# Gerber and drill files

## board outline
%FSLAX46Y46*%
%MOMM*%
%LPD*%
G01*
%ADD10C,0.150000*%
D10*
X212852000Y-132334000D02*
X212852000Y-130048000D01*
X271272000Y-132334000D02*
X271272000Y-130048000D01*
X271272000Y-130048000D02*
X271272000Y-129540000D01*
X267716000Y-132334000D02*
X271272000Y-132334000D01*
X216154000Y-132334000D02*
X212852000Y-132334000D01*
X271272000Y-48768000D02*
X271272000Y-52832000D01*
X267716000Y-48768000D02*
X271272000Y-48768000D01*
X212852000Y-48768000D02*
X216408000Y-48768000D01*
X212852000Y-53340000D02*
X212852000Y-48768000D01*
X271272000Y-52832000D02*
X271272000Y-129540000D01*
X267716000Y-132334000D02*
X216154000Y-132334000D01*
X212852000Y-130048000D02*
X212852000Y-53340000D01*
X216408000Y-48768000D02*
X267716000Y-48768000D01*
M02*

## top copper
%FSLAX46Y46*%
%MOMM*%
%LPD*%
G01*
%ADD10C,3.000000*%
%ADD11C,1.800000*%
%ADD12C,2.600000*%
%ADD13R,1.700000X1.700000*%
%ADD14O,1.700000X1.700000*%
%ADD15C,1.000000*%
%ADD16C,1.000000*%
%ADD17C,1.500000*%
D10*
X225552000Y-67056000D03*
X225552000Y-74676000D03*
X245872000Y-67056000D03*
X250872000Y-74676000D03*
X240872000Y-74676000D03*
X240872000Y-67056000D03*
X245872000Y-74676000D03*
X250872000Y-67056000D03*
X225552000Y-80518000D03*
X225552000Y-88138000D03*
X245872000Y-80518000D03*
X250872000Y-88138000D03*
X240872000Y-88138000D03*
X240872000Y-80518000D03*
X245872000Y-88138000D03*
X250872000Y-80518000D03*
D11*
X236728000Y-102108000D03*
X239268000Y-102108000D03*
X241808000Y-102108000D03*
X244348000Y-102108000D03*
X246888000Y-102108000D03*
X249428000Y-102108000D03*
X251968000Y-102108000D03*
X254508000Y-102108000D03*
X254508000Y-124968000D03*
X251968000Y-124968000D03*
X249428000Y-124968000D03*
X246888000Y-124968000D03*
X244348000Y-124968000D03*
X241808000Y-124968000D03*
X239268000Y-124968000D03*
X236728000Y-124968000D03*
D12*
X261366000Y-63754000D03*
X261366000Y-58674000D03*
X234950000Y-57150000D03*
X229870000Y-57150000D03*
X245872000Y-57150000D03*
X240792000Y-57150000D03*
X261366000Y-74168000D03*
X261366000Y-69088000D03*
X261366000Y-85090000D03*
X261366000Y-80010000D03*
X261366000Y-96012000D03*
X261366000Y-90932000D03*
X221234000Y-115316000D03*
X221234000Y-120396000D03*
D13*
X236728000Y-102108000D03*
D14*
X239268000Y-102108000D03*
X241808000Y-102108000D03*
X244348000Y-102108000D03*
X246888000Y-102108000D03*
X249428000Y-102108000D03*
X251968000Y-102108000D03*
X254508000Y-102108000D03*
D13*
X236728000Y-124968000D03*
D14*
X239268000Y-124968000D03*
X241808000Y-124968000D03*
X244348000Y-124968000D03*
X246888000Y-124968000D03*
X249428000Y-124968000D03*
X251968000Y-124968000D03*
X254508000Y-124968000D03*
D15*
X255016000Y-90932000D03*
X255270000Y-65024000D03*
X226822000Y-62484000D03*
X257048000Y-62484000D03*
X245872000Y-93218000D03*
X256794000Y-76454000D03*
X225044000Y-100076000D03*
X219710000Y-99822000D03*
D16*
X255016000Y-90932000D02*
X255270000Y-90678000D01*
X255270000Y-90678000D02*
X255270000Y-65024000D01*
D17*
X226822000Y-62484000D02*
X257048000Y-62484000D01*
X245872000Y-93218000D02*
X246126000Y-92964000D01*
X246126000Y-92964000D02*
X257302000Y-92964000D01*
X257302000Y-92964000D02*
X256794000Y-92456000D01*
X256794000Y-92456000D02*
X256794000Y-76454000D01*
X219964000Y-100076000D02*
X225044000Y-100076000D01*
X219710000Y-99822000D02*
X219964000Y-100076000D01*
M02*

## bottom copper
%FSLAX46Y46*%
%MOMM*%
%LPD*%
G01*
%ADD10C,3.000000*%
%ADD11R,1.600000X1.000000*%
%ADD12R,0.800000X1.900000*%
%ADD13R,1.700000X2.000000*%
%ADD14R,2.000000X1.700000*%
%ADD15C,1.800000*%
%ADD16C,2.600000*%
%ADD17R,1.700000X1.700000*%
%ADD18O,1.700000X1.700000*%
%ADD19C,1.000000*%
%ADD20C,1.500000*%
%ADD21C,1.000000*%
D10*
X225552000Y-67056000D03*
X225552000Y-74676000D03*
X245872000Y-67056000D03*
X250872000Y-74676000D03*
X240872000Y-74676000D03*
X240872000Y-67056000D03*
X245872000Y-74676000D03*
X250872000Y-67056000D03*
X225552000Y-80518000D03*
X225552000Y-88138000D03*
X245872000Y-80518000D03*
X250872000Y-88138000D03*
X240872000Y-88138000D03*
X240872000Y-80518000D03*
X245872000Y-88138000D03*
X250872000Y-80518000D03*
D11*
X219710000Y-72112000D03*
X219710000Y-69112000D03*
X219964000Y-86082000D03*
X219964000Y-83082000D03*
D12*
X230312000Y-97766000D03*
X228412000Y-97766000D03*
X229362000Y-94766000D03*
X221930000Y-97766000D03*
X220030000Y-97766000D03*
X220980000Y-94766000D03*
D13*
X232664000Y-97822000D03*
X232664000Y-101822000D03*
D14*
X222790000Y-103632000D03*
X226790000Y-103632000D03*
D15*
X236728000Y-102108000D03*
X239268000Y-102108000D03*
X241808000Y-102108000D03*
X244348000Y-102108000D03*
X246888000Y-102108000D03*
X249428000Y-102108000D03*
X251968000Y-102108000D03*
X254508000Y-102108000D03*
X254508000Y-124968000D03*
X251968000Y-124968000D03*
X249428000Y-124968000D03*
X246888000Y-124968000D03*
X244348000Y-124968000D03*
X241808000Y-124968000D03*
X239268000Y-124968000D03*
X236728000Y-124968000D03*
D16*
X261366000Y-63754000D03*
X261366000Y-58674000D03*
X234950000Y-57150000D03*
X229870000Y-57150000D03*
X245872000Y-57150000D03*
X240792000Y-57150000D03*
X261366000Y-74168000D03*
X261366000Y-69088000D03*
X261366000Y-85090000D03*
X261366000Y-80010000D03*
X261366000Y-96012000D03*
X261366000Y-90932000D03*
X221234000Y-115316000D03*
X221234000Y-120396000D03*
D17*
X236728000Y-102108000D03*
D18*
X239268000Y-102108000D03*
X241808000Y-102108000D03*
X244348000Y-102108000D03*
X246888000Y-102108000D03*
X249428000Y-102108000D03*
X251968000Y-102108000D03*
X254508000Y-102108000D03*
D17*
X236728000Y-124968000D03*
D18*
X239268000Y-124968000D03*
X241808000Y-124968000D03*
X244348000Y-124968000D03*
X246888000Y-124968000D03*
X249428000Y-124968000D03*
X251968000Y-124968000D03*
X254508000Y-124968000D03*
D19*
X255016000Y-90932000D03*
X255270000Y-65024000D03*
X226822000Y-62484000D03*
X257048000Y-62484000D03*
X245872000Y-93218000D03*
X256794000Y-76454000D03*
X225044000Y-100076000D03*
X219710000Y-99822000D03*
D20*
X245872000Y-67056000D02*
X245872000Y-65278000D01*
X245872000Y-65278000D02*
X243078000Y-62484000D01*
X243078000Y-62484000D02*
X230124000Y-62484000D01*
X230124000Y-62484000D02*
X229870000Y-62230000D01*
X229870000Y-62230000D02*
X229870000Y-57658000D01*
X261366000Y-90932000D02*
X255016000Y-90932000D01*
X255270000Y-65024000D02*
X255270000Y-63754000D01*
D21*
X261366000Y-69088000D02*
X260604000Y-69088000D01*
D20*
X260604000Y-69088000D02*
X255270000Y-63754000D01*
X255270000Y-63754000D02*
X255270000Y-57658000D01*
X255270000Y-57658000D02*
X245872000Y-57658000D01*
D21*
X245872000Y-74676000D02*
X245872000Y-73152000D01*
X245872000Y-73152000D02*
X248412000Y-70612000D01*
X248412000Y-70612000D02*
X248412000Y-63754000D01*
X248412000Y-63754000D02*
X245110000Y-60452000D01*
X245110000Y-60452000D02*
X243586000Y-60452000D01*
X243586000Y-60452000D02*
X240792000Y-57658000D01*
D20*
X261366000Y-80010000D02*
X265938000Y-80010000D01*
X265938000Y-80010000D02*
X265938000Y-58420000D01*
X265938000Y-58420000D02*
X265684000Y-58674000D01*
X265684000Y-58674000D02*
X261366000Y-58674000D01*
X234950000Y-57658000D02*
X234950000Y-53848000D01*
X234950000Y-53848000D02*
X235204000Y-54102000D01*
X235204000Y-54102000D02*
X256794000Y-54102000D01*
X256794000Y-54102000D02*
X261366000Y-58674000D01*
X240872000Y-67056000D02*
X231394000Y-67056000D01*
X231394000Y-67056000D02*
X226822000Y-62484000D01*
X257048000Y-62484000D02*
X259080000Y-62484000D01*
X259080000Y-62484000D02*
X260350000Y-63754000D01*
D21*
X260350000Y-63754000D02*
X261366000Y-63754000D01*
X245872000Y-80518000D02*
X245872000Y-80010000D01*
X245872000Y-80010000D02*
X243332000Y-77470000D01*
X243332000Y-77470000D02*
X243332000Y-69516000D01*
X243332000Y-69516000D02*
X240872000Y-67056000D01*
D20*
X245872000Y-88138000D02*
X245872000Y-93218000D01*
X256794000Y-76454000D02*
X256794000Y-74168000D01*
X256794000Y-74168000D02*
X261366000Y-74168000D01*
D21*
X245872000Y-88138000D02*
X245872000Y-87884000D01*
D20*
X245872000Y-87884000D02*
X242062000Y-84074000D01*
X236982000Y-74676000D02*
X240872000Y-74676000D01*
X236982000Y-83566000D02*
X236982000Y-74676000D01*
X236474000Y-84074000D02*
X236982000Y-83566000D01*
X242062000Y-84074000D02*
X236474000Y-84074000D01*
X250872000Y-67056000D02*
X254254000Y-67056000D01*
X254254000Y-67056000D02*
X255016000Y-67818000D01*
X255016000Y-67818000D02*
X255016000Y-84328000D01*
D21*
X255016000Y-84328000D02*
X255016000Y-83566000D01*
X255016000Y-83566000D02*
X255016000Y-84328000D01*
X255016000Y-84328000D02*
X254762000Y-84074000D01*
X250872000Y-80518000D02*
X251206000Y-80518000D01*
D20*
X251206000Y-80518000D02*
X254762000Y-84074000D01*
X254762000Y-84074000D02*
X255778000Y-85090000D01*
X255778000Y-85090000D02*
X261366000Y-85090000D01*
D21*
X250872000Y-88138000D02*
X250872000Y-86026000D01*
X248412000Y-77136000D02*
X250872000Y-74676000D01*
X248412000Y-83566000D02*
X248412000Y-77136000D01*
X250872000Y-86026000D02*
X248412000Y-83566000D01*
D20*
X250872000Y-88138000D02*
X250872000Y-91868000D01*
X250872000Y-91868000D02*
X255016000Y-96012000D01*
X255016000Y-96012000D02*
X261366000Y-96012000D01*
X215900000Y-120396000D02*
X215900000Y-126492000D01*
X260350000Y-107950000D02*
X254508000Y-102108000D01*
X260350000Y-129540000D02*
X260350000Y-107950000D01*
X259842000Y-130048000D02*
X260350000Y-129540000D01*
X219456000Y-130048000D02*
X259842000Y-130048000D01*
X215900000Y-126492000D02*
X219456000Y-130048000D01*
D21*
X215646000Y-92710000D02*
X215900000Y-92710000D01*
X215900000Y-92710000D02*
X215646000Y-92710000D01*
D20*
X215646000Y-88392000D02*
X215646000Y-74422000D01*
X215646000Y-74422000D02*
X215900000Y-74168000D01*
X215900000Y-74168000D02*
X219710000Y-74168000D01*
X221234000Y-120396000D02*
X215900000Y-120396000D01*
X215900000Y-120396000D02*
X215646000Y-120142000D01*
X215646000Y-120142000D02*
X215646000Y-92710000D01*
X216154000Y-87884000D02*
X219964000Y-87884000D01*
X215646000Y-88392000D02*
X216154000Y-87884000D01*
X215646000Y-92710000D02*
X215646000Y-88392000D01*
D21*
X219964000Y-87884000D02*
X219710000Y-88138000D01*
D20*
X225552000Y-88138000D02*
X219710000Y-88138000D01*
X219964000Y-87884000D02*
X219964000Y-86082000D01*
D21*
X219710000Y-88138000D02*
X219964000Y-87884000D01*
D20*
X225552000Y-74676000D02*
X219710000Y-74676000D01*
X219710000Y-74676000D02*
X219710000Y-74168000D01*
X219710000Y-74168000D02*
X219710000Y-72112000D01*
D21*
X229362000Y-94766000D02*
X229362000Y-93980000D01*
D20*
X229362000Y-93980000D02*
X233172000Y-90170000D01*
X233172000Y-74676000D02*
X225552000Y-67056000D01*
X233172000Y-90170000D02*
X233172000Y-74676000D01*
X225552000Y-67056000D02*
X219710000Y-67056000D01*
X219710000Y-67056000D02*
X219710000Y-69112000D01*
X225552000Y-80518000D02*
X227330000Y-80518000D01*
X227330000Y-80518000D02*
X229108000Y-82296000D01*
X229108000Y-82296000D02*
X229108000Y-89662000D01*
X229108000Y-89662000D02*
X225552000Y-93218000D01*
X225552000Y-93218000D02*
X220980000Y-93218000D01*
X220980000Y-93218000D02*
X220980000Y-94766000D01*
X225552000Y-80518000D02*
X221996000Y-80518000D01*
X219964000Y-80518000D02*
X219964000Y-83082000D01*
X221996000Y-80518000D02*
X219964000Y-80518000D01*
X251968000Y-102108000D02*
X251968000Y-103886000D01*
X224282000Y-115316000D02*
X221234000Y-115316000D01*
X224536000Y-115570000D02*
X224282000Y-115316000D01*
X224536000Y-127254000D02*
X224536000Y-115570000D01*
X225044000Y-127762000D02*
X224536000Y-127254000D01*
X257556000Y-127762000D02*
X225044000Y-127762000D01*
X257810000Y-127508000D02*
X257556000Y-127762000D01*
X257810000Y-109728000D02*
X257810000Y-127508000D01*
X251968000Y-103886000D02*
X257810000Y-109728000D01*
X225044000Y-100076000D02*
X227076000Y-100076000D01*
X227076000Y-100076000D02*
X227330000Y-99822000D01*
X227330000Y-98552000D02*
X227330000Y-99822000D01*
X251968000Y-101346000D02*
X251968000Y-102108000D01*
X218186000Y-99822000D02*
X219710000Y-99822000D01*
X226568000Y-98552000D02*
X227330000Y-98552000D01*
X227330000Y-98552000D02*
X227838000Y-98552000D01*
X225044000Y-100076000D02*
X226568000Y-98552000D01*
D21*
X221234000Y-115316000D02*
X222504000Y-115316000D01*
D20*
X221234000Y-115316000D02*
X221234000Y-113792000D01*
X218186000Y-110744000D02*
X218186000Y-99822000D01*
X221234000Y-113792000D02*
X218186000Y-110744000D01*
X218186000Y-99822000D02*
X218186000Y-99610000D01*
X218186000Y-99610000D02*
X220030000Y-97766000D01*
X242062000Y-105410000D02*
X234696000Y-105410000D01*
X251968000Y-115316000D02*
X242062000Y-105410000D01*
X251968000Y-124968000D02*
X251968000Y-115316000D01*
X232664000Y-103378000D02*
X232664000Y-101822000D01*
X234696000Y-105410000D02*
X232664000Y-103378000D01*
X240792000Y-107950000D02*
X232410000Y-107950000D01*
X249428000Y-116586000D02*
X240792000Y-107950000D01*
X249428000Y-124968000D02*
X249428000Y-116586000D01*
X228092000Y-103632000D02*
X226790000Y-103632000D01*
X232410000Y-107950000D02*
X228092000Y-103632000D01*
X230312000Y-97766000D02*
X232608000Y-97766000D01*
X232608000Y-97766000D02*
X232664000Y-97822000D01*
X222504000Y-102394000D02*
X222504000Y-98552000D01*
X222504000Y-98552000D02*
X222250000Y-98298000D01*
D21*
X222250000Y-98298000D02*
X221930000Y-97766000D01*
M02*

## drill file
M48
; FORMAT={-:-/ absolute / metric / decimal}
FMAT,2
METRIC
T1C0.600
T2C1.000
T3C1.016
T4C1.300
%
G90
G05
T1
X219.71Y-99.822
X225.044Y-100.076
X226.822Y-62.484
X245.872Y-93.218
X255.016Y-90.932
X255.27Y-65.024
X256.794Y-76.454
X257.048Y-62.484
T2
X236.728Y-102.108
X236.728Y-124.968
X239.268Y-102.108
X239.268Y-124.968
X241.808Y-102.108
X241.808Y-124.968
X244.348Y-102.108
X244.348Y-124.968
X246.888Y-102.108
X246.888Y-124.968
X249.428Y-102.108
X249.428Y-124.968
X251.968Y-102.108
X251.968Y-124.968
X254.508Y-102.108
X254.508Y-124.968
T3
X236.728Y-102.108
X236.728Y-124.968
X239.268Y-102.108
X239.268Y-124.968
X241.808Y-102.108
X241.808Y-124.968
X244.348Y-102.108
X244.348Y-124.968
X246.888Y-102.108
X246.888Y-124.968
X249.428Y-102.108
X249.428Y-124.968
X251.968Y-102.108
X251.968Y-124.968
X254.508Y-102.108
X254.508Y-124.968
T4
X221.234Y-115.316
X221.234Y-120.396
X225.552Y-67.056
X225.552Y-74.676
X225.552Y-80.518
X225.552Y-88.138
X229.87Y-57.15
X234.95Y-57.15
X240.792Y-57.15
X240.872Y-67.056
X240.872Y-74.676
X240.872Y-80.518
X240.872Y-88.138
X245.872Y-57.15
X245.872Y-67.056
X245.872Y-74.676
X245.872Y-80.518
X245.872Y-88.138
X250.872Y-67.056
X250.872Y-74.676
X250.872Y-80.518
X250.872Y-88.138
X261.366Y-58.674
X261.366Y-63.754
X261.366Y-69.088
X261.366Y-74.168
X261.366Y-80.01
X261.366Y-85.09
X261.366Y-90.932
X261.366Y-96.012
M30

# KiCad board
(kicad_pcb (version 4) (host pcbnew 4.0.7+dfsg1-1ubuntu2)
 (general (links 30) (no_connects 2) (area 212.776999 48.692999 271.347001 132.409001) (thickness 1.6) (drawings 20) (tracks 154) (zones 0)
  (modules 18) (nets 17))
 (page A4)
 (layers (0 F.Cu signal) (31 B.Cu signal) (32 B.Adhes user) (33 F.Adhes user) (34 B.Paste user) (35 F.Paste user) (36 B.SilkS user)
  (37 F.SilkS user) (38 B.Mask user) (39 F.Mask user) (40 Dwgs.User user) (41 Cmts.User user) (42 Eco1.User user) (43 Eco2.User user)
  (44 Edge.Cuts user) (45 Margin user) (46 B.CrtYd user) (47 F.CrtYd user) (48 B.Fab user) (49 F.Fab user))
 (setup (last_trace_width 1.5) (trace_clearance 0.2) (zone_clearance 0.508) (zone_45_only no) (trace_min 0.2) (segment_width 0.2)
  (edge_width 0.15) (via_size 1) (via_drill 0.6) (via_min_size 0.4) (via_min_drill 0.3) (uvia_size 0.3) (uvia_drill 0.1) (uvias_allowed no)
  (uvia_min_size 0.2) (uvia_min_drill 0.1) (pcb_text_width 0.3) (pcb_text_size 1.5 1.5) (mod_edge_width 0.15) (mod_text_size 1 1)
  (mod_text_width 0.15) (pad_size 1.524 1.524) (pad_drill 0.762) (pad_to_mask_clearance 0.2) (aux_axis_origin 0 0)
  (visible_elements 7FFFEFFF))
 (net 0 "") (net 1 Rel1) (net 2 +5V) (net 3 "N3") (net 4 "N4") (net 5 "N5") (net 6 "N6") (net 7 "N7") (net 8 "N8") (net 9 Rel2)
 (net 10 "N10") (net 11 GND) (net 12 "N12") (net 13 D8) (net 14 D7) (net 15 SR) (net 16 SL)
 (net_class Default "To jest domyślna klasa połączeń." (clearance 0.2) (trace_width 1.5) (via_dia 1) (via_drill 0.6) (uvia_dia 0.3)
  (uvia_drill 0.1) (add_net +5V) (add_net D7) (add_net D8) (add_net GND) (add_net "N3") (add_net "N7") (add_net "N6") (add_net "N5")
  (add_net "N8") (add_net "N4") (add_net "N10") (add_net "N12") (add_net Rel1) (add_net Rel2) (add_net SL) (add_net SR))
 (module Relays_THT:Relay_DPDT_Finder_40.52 (layer F.Cu) (at 225.552 67.056)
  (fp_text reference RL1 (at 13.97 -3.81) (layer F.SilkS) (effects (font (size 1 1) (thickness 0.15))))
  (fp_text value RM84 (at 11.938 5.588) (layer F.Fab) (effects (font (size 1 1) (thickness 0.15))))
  (pad A1 thru_hole circle (at 0 0) (size 3 3) (drill 1.3) (layers *.Cu *.Mask) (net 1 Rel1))
  (pad A2 thru_hole circle (at 0 7.62) (size 3 3) (drill 1.3) (layers *.Cu *.Mask) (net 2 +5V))
  (pad 11 thru_hole circle (at 20.32 0) (size 3 3) (drill 1.3) (layers *.Cu *.Mask) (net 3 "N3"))
  (pad 24 thru_hole circle (at 25.32 7.62) (size 3 3) (drill 1.3) (layers *.Cu *.Mask) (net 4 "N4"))
  (pad 22 thru_hole circle (at 15.32 7.62) (size 3 3) (drill 1.3) (layers *.Cu *.Mask) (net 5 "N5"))
  (pad 12 thru_hole circle (at 15.32 0) (size 3 3) (drill 1.3) (layers *.Cu *.Mask) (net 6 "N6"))
  (pad 21 thru_hole circle (at 20.32 7.62) (size 3 3) (drill 1.3) (layers *.Cu *.Mask) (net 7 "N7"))
  (pad 14 thru_hole circle (at 25.32 0) (size 3 3) (drill 1.3) (layers *.Cu *.Mask) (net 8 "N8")))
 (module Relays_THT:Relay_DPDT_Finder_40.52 (layer F.Cu) (at 225.552 80.518)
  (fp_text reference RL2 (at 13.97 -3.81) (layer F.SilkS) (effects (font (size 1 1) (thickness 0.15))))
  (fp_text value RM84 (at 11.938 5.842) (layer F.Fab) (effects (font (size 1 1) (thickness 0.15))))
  (pad A1 thru_hole circle (at 0 0) (size 3 3) (drill 1.3) (layers *.Cu *.Mask) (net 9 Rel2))
  (pad A2 thru_hole circle (at 0 7.62) (size 3 3) (drill 1.3) (layers *.Cu *.Mask) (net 2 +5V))
  (pad 11 thru_hole circle (at 20.32 0) (size 3 3) (drill 1.3) (layers *.Cu *.Mask) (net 6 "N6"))
  (pad 24 thru_hole circle (at 25.32 7.62) (size 3 3) (drill 1.3) (layers *.Cu *.Mask) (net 4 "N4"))
  (pad 22 thru_hole circle (at 15.32 7.62) (size 3 3) (drill 1.3) (layers *.Cu *.Mask))
  (pad 12 thru_hole circle (at 15.32 0) (size 3 3) (drill 1.3) (layers *.Cu *.Mask))
  (pad 21 thru_hole circle (at 20.32 7.62) (size 3 3) (drill 1.3) (layers *.Cu *.Mask) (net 5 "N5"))
  (pad 14 thru_hole circle (at 25.32 0) (size 3 3) (drill 1.3) (layers *.Cu *.Mask) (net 8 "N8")))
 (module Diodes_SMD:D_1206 (layer B.Cu) (at 219.71 70.612 90)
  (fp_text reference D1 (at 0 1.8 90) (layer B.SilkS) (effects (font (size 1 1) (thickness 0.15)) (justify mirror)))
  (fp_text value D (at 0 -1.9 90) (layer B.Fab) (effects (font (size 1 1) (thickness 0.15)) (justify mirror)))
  (pad 1 smd rect (at -1.5 0 90) (size 1 1.6) (layers B.Cu B.Paste B.Mask) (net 2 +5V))
  (pad 2 smd rect (at 1.5 0 90) (size 1 1.6) (layers B.Cu B.Paste B.Mask) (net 1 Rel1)))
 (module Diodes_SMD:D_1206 (layer B.Cu) (at 219.964 84.582 90)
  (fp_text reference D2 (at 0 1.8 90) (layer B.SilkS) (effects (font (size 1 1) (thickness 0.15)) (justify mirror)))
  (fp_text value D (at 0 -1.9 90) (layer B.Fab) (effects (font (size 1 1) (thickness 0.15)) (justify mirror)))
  (pad 1 smd rect (at -1.5 0 90) (size 1 1.6) (layers B.Cu B.Paste B.Mask) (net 2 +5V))
  (pad 2 smd rect (at 1.5 0 90) (size 1 1.6) (layers B.Cu B.Paste B.Mask) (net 9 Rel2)))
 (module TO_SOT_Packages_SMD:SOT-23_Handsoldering (layer B.Cu) (at 229.362 96.266 90)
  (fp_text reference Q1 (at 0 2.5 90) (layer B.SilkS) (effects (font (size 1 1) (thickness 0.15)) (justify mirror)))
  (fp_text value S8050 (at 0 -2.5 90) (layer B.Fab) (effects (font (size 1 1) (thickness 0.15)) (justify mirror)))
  (pad 1 smd rect (at -1.5 0.95 90) (size 1.9 0.8) (layers B.Cu B.Paste B.Mask) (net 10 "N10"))
  (pad 2 smd rect (at -1.5 -0.95 90) (size 1.9 0.8) (layers B.Cu B.Paste B.Mask) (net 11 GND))
  (pad 3 smd rect (at 1.5 0 90) (size 1.9 0.8) (layers B.Cu B.Paste B.Mask) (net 1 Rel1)))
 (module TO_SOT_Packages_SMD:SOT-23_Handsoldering (layer B.Cu) (at 220.98 96.266 90)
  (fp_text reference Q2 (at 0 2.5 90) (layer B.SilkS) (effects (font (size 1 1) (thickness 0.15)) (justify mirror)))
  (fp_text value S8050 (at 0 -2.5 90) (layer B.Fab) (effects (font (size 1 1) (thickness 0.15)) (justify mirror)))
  (pad 1 smd rect (at -1.5 0.95 90) (size 1.9 0.8) (layers B.Cu B.Paste B.Mask) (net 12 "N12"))
  (pad 2 smd rect (at -1.5 -0.95 90) (size 1.9 0.8) (layers B.Cu B.Paste B.Mask) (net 11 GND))
  (pad 3 smd rect (at 1.5 0 90) (size 1.9 0.8) (layers B.Cu B.Paste B.Mask) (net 9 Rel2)))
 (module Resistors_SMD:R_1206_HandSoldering (layer B.Cu) (at 232.664 99.822 270)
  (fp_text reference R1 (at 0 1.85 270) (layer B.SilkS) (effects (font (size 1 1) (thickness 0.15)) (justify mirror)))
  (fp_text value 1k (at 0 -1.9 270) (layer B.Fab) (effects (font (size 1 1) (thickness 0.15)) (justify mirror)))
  (pad 1 smd rect (at -2 0 270) (size 2 1.7) (layers B.Cu B.Paste B.Mask) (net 10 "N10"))
  (pad 2 smd rect (at 2 0 270) (size 2 1.7) (layers B.Cu B.Paste B.Mask) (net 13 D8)))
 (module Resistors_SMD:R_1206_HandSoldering (layer B.Cu) (at 224.79 103.632)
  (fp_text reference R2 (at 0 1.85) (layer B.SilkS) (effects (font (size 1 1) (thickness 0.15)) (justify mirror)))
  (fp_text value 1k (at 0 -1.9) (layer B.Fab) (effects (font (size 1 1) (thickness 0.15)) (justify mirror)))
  (pad 1 smd rect (at -2 0) (size 2 1.7) (layers B.Cu B.Paste B.Mask) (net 12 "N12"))
  (pad 2 smd rect (at 2 0) (size 2 1.7) (layers B.Cu B.Paste B.Mask) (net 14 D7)))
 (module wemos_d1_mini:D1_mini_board (layer B.Cu) (at 246.888 113.538 270)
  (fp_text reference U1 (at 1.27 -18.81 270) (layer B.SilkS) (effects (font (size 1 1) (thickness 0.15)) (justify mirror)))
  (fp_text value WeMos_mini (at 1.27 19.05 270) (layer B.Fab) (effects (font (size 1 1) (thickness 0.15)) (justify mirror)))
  (pad 8 thru_hole circle (at -11.43 10.16 270) (size 1.8 1.8) (drill 1.016) (layers *.Cu *.Mask B.SilkS))
  (pad 7 thru_hole circle (at -11.43 7.62 270) (size 1.8 1.8) (drill 1.016) (layers *.Cu *.Mask B.SilkS))
  (pad 6 thru_hole circle (at -11.43 5.08 270) (size 1.8 1.8) (drill 1.016) (layers *.Cu *.Mask B.SilkS))
  (pad 5 thru_hole circle (at -11.43 2.54 270) (size 1.8 1.8) (drill 1.016) (layers *.Cu *.Mask B.SilkS))
  (pad 4 thru_hole circle (at -11.43 0 270) (size 1.8 1.8) (drill 1.016) (layers *.Cu *.Mask B.SilkS))
  (pad 3 thru_hole circle (at -11.43 -2.54 270) (size 1.8 1.8) (drill 1.016) (layers *.Cu *.Mask B.SilkS))
  (pad 2 thru_hole circle (at -11.43 -5.08 270) (size 1.8 1.8) (drill 1.016) (layers *.Cu *.Mask B.SilkS) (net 11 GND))
  (pad 1 thru_hole circle (at -11.43 -7.62 270) (size 1.8 1.8) (drill 1.016) (layers *.Cu *.Mask B.SilkS) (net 2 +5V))
  (pad 16 thru_hole circle (at 11.43 -7.62 270) (size 1.8 1.8) (drill 1.016) (layers *.Cu *.Mask B.SilkS))
  (pad 15 thru_hole circle (at 11.43 -5.08 270) (size 1.8 1.8) (drill 1.016) (layers *.Cu *.Mask B.SilkS) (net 13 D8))
  (pad 14 thru_hole circle (at 11.43 -2.54 270) (size 1.8 1.8) (drill 1.016) (layers *.Cu *.Mask B.SilkS) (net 14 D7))
  (pad 13 thru_hole circle (at 11.43 0 270) (size 1.8 1.8) (drill 1.016) (layers *.Cu *.Mask B.SilkS))
  (pad 12 thru_hole circle (at 11.43 2.54 270) (size 1.8 1.8) (drill 1.016) (layers *.Cu *.Mask B.SilkS))
  (pad 11 thru_hole circle (at 11.43 5.08 270) (size 1.8 1.8) (drill 1.016) (layers *.Cu *.Mask B.SilkS))
  (pad 10 thru_hole circle (at 11.43 7.62 270) (size 1.8 1.8) (drill 1.016) (layers *.Cu *.Mask B.SilkS))
  (pad 9 thru_hole circle (at 11.43 10.16 270) (size 1.8 1.8) (drill 1.016) (layers *.Cu *.Mask B.SilkS)))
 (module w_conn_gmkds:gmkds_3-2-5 (layer F.Cu) (at 261.366 61.214 90)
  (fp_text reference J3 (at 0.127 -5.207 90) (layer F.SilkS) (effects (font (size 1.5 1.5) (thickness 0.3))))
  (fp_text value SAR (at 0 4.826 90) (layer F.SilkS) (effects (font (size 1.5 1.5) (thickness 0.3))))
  (pad 1 thru_hole circle (at -2.54 0 90) (size 2.6 2.6) (drill 1.3) (layers *.Cu *.Mask F.SilkS) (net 6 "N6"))
  (pad 2 thru_hole circle (at 2.54 0 90) (size 2.6 2.6) (drill 1.3) (layers *.Cu *.Mask F.SilkS) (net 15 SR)))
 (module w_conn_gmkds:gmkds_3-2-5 (layer F.Cu) (at 232.41 57.15 180)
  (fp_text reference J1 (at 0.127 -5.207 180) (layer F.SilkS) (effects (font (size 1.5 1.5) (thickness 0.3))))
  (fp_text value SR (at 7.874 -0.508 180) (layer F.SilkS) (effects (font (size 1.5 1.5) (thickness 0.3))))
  (pad 1 thru_hole circle (at -2.54 0 180) (size 2.6 2.6) (drill 1.3) (layers *.Cu *.Mask F.SilkS) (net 15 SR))
  (pad 2 thru_hole circle (at 2.54 0 180) (size 2.6 2.6) (drill 1.3) (layers *.Cu *.Mask F.SilkS) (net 3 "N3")))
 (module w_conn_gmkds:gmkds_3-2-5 (layer F.Cu) (at 243.332 57.15 180)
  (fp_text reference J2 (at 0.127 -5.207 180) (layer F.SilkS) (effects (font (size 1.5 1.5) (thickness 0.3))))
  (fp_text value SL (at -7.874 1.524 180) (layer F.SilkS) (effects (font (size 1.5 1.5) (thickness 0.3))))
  (pad 1 thru_hole circle (at -2.54 0 180) (size 2.6 2.6) (drill 1.3) (layers *.Cu *.Mask F.SilkS) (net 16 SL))
  (pad 2 thru_hole circle (at 2.54 0 180) (size 2.6 2.6) (drill 1.3) (layers *.Cu *.Mask F.SilkS) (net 7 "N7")))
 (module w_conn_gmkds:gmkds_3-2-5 (layer F.Cu) (at 261.366 71.628 90)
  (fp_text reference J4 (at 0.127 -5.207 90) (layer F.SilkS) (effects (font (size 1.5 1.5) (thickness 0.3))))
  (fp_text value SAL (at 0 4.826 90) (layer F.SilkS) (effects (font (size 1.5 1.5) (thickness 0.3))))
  (pad 1 thru_hole circle (at -2.54 0 90) (size 2.6 2.6) (drill 1.3) (layers *.Cu *.Mask F.SilkS) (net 5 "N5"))
  (pad 2 thru_hole circle (at 2.54 0 90) (size 2.6 2.6) (drill 1.3) (layers *.Cu *.Mask F.SilkS) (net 16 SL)))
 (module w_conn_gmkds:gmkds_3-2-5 (layer F.Cu) (at 261.366 82.55 90)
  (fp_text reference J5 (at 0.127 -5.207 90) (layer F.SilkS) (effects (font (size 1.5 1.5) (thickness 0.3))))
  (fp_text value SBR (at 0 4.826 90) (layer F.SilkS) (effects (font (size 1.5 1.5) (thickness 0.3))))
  (pad 1 thru_hole circle (at -2.54 0 90) (size 2.6 2.6) (drill 1.3) (layers *.Cu *.Mask F.SilkS) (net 8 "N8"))
  (pad 2 thru_hole circle (at 2.54 0 90) (size 2.6 2.6) (drill 1.3) (layers *.Cu *.Mask F.SilkS) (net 15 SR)))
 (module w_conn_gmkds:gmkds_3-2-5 (layer F.Cu) (at 261.366 93.472 90)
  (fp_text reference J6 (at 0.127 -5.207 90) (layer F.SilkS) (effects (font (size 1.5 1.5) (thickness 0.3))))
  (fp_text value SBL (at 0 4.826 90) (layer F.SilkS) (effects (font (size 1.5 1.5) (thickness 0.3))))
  (pad 1 thru_hole circle (at -2.54 0 90) (size 2.6 2.6) (drill 1.3) (layers *.Cu *.Mask F.SilkS) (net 4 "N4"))
  (pad 2 thru_hole circle (at 2.54 0 90) (size 2.6 2.6) (drill 1.3) (layers *.Cu *.Mask F.SilkS) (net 16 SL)))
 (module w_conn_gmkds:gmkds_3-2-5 (layer F.Cu) (at 221.234 117.856 270)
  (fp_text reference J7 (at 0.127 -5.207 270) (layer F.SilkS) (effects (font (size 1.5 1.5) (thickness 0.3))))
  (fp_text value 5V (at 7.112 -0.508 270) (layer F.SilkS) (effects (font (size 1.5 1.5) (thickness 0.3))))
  (pad 1 thru_hole circle (at -2.54 0 270) (size 2.6 2.6) (drill 1.3) (layers *.Cu *.Mask F.SilkS) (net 11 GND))
  (pad 2 thru_hole circle (at 2.54 0 270) (size 2.6 2.6) (drill 1.3) (layers *.Cu *.Mask F.SilkS) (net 2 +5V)))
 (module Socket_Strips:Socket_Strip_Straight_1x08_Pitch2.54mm (layer F.Cu) (at 236.728 102.108 90)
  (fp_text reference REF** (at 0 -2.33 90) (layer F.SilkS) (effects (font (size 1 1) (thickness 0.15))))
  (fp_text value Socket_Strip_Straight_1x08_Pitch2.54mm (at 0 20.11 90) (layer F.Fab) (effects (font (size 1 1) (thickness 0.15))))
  (pad 1 thru_hole rect (at 0 0 90) (size 1.7 1.7) (drill 1) (layers *.Cu *.Mask))
  (pad 2 thru_hole oval (at 0 2.54 90) (size 1.7 1.7) (drill 1) (layers *.Cu *.Mask))
  (pad 3 thru_hole oval (at 0 5.08 90) (size 1.7 1.7) (drill 1) (layers *.Cu *.Mask))
  (pad 4 thru_hole oval (at 0 7.62 90) (size 1.7 1.7) (drill 1) (layers *.Cu *.Mask))
  (pad 5 thru_hole oval (at 0 10.16 90) (size 1.7 1.7) (drill 1) (layers *.Cu *.Mask))
  (pad 6 thru_hole oval (at 0 12.7 90) (size 1.7 1.7) (drill 1) (layers *.Cu *.Mask))
  (pad 7 thru_hole oval (at 0 15.24 90) (size 1.7 1.7) (drill 1) (layers *.Cu *.Mask))
  (pad 8 thru_hole oval (at 0 17.78 90) (size 1.7 1.7) (drill 1) (layers *.Cu *.Mask)))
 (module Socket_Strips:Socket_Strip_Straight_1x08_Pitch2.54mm (layer F.Cu) (at 236.728 124.968 90)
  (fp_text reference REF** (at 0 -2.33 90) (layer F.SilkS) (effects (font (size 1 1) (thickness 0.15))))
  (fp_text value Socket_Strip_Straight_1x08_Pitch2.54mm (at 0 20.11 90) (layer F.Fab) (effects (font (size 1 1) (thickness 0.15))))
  (pad 1 thru_hole rect (at 0 0 90) (size 1.7 1.7) (drill 1) (layers *.Cu *.Mask))
  (pad 2 thru_hole oval (at 0 2.54 90) (size 1.7 1.7) (drill 1) (layers *.Cu *.Mask))
  (pad 3 thru_hole oval (at 0 5.08 90) (size 1.7 1.7) (drill 1) (layers *.Cu *.Mask))
  (pad 4 thru_hole oval (at 0 7.62 90) (size 1.7 1.7) (drill 1) (layers *.Cu *.Mask))
  (pad 5 thru_hole oval (at 0 10.16 90) (size 1.7 1.7) (drill 1) (layers *.Cu *.Mask))
  (pad 6 thru_hole oval (at 0 12.7 90) (size 1.7 1.7) (drill 1) (layers *.Cu *.Mask))
  (pad 7 thru_hole oval (at 0 15.24 90) (size 1.7 1.7) (drill 1) (layers *.Cu *.Mask))
  (pad 8 thru_hole oval (at 0 17.78 90) (size 1.7 1.7) (drill 1) (layers *.Cu *.Mask)))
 (gr_line (start 212.852 132.334) (end 212.852 130.048) (angle 90) (layer Edge.Cuts) (width 0.15))
 (gr_line (start 271.272 132.334) (end 271.272 130.048) (angle 90) (layer Edge.Cuts) (width 0.15))
 (gr_line (start 271.272 130.048) (end 271.272 129.54) (angle 90) (layer Edge.Cuts) (width 0.15))
 (gr_line (start 267.716 132.334) (end 271.272 132.334) (angle 90) (layer Edge.Cuts) (width 0.15))
 (gr_line (start 216.154 132.334) (end 212.852 132.334) (angle 90) (layer Edge.Cuts) (width 0.15))
 (gr_line (start 271.272 48.768) (end 271.272 52.832) (angle 90) (layer Edge.Cuts) (width 0.15))
 (gr_line (start 267.716 48.768) (end 271.272 48.768) (angle 90) (layer Edge.Cuts) (width 0.15))
 (gr_line (start 212.852 48.768) (end 216.408 48.768) (angle 90) (layer Edge.Cuts) (width 0.15))
 (gr_line (start 212.852 53.34) (end 212.852 48.768) (angle 90) (layer Edge.Cuts) (width 0.15))
 (gr_line (start 271.272 52.832) (end 271.272 129.54) (angle 90) (layer Edge.Cuts) (width 0.15))
 (gr_line (start 267.716 132.334) (end 216.154 132.334) (angle 90) (layer Edge.Cuts) (width 0.15))
 (gr_line (start 212.852 130.048) (end 212.852 53.34) (angle 90) (layer Edge.Cuts) (width 0.15))
 (gr_line (start 216.408 48.768) (end 267.716 48.768) (angle 90) (layer Edge.Cuts) (width 0.15))
 (segment (start 245.872 67.056) (end 245.872 65.278) (width 1.5) (layer B.Cu) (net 3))
 (segment (start 245.872 65.278) (end 243.078 62.484) (width 1.5) (layer B.Cu) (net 3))
 (segment (start 243.078 62.484) (end 230.124 62.484) (width 1.5) (layer B.Cu) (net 3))
 (segment (start 230.124 62.484) (end 229.87 62.23) (width 1.5) (layer B.Cu) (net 3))
 (segment (start 229.87 62.23) (end 229.87 57.658) (width 1.5) (layer B.Cu) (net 3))
 (segment (start 261.366 90.932) (end 255.016 90.932) (width 1.5) (layer B.Cu) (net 16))
 (via (at 255.016 90.932) (size 1) (drill 0.6) (layers F.Cu B.Cu) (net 16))
 (segment (start 255.016 90.932) (end 255.27 90.678) (width 1) (layer F.Cu) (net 16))
 (segment (start 255.27 90.678) (end 255.27 65.024) (width 1) (layer F.Cu) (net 16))
 (via (at 255.27 65.024) (size 1) (drill 0.6) (layers F.Cu B.Cu) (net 16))
 (segment (start 255.27 65.024) (end 255.27 63.754) (width 1.5) (layer B.Cu) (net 16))
 (segment (start 261.366 69.088) (end 260.604 69.088) (width 1) (layer B.Cu) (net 16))
 (segment (start 260.604 69.088) (end 255.27 63.754) (width 1.5) (layer B.Cu) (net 16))
 (segment (start 255.27 63.754) (end 255.27 57.658) (width 1.5) (layer B.Cu) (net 16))
 (segment (start 255.27 57.658) (end 245.872 57.658) (width 1.5) (layer B.Cu) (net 16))
 (segment (start 245.872 74.676) (end 245.872 73.152) (width 1) (layer B.Cu) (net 7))
 (segment (start 245.872 73.152) (end 248.412 70.612) (width 1) (layer B.Cu) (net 7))
 (segment (start 248.412 70.612) (end 248.412 63.754) (width 1) (layer B.Cu) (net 7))
 (segment (start 248.412 63.754) (end 245.11 60.452) (width 1) (layer B.Cu) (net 7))
 (segment (start 245.11 60.452) (end 243.586 60.452) (width 1) (layer B.Cu) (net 7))
 (segment (start 243.586 60.452) (end 240.792 57.658) (width 1) (layer B.Cu) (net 7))
 (segment (start 261.366 80.01) (end 265.938 80.01) (width 1.5) (layer B.Cu) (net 15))
 (segment (start 265.938 80.01) (end 265.938 58.42) (width 1.5) (layer B.Cu) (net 15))
 (segment (start 265.938 58.42) (end 265.684 58.674) (width 1.5) (layer B.Cu) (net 15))
 (segment (start 265.684 58.674) (end 261.366 58.674) (width 1.5) (layer B.Cu) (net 15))
 (segment (start 234.95 57.658) (end 234.95 53.848) (width 1.5) (layer B.Cu) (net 15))
 (segment (start 234.95 53.848) (end 235.204 54.102) (width 1.5) (layer B.Cu) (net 15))
 (segment (start 235.204 54.102) (end 256.794 54.102) (width 1.5) (layer B.Cu) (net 15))
 (segment (start 256.794 54.102) (end 261.366 58.674) (width 1.5) (layer B.Cu) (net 15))
 (segment (start 240.872 67.056) (end 231.394 67.056) (width 1.5) (layer B.Cu) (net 6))
 (segment (start 231.394 67.056) (end 226.822 62.484) (width 1.5) (layer B.Cu) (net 6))
 (via (at 226.822 62.484) (size 1) (drill 0.6) (layers F.Cu B.Cu) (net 6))
 (segment (start 226.822 62.484) (end 257.048 62.484) (width 1.5) (layer F.Cu) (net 6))
 (via (at 257.048 62.484) (size 1) (drill 0.6) (layers F.Cu B.Cu) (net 6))
 (segment (start 257.048 62.484) (end 259.08 62.484) (width 1.5) (layer B.Cu) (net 6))
 (segment (start 259.08 62.484) (end 260.35 63.754) (width 1.5) (layer B.Cu) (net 6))
 (segment (start 260.35 63.754) (end 261.366 63.754) (width 1) (layer B.Cu) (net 6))
 (segment (start 245.872 80.518) (end 245.872 80.01) (width 1) (layer B.Cu) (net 6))
 (segment (start 245.872 80.01) (end 243.332 77.47) (width 1) (layer B.Cu) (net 6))
 (segment (start 243.332 77.47) (end 243.332 69.516) (width 1) (layer B.Cu) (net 6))
 (segment (start 243.332 69.516) (end 240.872 67.056) (width 1) (layer B.Cu) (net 6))
 (segment (start 245.872 88.138) (end 245.872 93.218) (width 1.5) (layer B.Cu) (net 5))
 (via (at 245.872 93.218) (size 1) (drill 0.6) (layers F.Cu B.Cu) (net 5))
 (segment (start 245.872 93.218) (end 246.126 92.964) (width 1.5) (layer F.Cu) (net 5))
 (segment (start 246.126 92.964) (end 257.302 92.964) (width 1.5) (layer F.Cu) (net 5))
 (segment (start 257.302 92.964) (end 256.794 92.456) (width 1.5) (layer F.Cu) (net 5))
 (segment (start 256.794 92.456) (end 256.794 76.454) (width 1.5) (layer F.Cu) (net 5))
 (via (at 256.794 76.454) (size 1) (drill 0.6) (layers F.Cu B.Cu) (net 5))
 (segment (start 256.794 76.454) (end 256.794 74.168) (width 1.5) (layer B.Cu) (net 5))
 (segment (start 256.794 74.168) (end 261.366 74.168) (width 1.5) (layer B.Cu) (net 5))
 (segment (start 245.872 88.138) (end 245.872 87.884) (width 1) (layer B.Cu) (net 5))
 (segment (start 245.872 87.884) (end 242.062 84.074) (width 1.5) (layer B.Cu) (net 5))
 (segment (start 236.982 74.676) (end 240.872 74.676) (width 1.5) (layer B.Cu) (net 5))
 (segment (start 236.982 83.566) (end 236.982 74.676) (width 1.5) (layer B.Cu) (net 5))
 (segment (start 236.474 84.074) (end 236.982 83.566) (width 1.5) (layer B.Cu) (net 5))
 (segment (start 242.062 84.074) (end 236.474 84.074) (width 1.5) (layer B.Cu) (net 5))
 (segment (start 250.872 67.056) (end 254.254 67.056) (width 1.5) (layer B.Cu) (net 8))
 (segment (start 254.254 67.056) (end 255.016 67.818) (width 1.5) (layer B.Cu) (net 8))
 (segment (start 255.016 67.818) (end 255.016 84.328) (width 1.5) (layer B.Cu) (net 8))
 (segment (start 255.016 84.328) (end 255.016 83.566) (width 1) (layer B.Cu) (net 8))
 (segment (start 255.016 83.566) (end 255.016 84.328) (width 1) (layer B.Cu) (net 8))
 (segment (start 255.016 84.328) (end 254.762 84.074) (width 1) (layer B.Cu) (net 8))
 (segment (start 250.872 80.518) (end 251.206 80.518) (width 1) (layer B.Cu) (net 8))
 (segment (start 251.206 80.518) (end 254.762 84.074) (width 1.5) (layer B.Cu) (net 8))
 (segment (start 254.762 84.074) (end 255.778 85.09) (width 1.5) (layer B.Cu) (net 8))
 (segment (start 255.778 85.09) (end 261.366 85.09) (width 1.5) (layer B.Cu) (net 8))
 (segment (start 250.872 88.138) (end 250.872 86.026) (width 1) (layer B.Cu) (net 4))
 (segment (start 248.412 77.136) (end 250.872 74.676) (width 1) (layer B.Cu) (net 4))
 (segment (start 248.412 83.566) (end 248.412 77.136) (width 1) (layer B.Cu) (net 4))
 (segment (start 250.872 86.026) (end 248.412 83.566) (width 1) (layer B.Cu) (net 4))
 (segment (start 250.872 88.138) (end 250.872 91.868) (width 1.5) (layer B.Cu) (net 4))
 (segment (start 250.872 91.868) (end 255.016 96.012) (width 1.5) (layer B.Cu) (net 4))
 (segment (start 255.016 96.012) (end 261.366 96.012) (width 1.5) (layer B.Cu) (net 4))
 (segment (start 215.9 120.396) (end 215.9 126.492) (width 1.5) (layer B.Cu) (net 2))
 (segment (start 260.35 107.95) (end 254.508 102.108) (width 1.5) (layer B.Cu) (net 2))
 (segment (start 260.35 129.54) (end 260.35 107.95) (width 1.5) (layer B.Cu) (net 2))
 (segment (start 259.842 130.048) (end 260.35 129.54) (width 1.5) (layer B.Cu) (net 2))
 (segment (start 219.456 130.048) (end 259.842 130.048) (width 1.5) (layer B.Cu) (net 2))
 (segment (start 215.9 126.492) (end 219.456 130.048) (width 1.5) (layer B.Cu) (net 2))
 (segment (start 215.646 92.71) (end 215.9 92.71) (width 1) (layer B.Cu) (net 2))
 (segment (start 215.9 92.71) (end 215.646 92.71) (width 1) (layer B.Cu) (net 2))
 (segment (start 215.646 88.392) (end 215.646 74.422) (width 1.5) (layer B.Cu) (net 2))
 (segment (start 215.646 74.422) (end 215.9 74.168) (width 1.5) (layer B.Cu) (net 2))
 (segment (start 215.9 74.168) (end 219.71 74.168) (width 1.5) (layer B.Cu) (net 2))
 (segment (start 221.234 120.396) (end 215.9 120.396) (width 1.5) (layer B.Cu) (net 2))
 (segment (start 215.9 120.396) (end 215.646 120.142) (width 1.5) (layer B.Cu) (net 2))
 (segment (start 215.646 120.142) (end 215.646 92.71) (width 1.5) (layer B.Cu) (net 2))
 (segment (start 216.154 87.884) (end 219.964 87.884) (width 1.5) (layer B.Cu) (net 2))
 (segment (start 215.646 88.392) (end 216.154 87.884) (width 1.5) (layer B.Cu) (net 2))
 (segment (start 215.646 92.71) (end 215.646 88.392) (width 1.5) (layer B.Cu) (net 2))
 (segment (start 219.964 87.884) (end 219.71 88.138) (width 1) (layer B.Cu) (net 2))
 (segment (start 225.552 88.138) (end 219.71 88.138) (width 1.5) (layer B.Cu) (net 2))
 (segment (start 219.964 87.884) (end 219.964 86.082) (width 1.5) (layer B.Cu) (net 2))
 (segment (start 219.71 88.138) (end 219.964 87.884) (width 1) (layer B.Cu) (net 2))
 (segment (start 225.552 74.676) (end 219.71 74.676) (width 1.5) (layer B.Cu) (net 2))
 (segment (start 219.71 74.676) (end 219.71 74.168) (width 1.5) (layer B.Cu) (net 2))
 (segment (start 219.71 74.168) (end 219.71 72.112) (width 1.5) (layer B.Cu) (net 2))
 (segment (start 229.362 94.766) (end 229.362 93.98) (width 1) (layer B.Cu) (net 1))
 (segment (start 229.362 93.98) (end 233.172 90.17) (width 1.5) (layer B.Cu) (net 1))
 (segment (start 233.172 74.676) (end 225.552 67.056) (width 1.5) (layer B.Cu) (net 1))
 (segment (start 233.172 90.17) (end 233.172 74.676) (width 1.5) (layer B.Cu) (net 1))
 (segment (start 225.552 67.056) (end 219.71 67.056) (width 1.5) (layer B.Cu) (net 1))
 (segment (start 219.71 67.056) (end 219.71 69.112) (width 1.5) (layer B.Cu) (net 1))
 (segment (start 225.552 80.518) (end 227.33 80.518) (width 1.5) (layer B.Cu) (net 9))
 (segment (start 227.33 80.518) (end 229.108 82.296) (width 1.5) (layer B.Cu) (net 9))
 (segment (start 229.108 82.296) (end 229.108 89.662) (width 1.5) (layer B.Cu) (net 9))
 (segment (start 229.108 89.662) (end 225.552 93.218) (width 1.5) (layer B.Cu) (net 9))
 (segment (start 225.552 93.218) (end 220.98 93.218) (width 1.5) (layer B.Cu) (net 9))
 (segment (start 220.98 93.218) (end 220.98 94.766) (width 1.5) (layer B.Cu) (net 9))
 (segment (start 225.552 80.518) (end 221.996 80.518) (width 1.5) (layer B.Cu) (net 9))
 (segment (start 219.964 80.518) (end 219.964 83.082) (width 1.5) (layer B.Cu) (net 9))
 (segment (start 221.996 80.518) (end 219.964 80.518) (width 1.5) (layer B.Cu) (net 9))
 (segment (start 251.968 102.108) (end 251.968 103.886) (width 1.5) (layer B.Cu) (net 11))
 (segment (start 224.282 115.316) (end 221.234 115.316) (width 1.5) (layer B.Cu) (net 11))
 (segment (start 224.536 115.57) (end 224.282 115.316) (width 1.5) (layer B.Cu) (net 11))
 (segment (start 224.536 127.254) (end 224.536 115.57) (width 1.5) (layer B.Cu) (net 11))
 (segment (start 225.044 127.762) (end 224.536 127.254) (width 1.5) (layer B.Cu) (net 11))
 (segment (start 257.556 127.762) (end 225.044 127.762) (width 1.5) (layer B.Cu) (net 11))
 (segment (start 257.81 127.508) (end 257.556 127.762) (width 1.5) (layer B.Cu) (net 11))
 (segment (start 257.81 109.728) (end 257.81 127.508) (width 1.5) (layer B.Cu) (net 11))
 (segment (start 251.968 103.886) (end 257.81 109.728) (width 1.5) (layer B.Cu) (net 11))
 (segment (start 225.044 100.076) (end 227.076 100.076) (width 1.5) (layer B.Cu) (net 11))
 (segment (start 227.076 100.076) (end 227.33 99.822) (width 1.5) (layer B.Cu) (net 11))
 (segment (start 227.33 98.552) (end 227.33 99.822) (width 1.5) (layer B.Cu) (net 11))
 (segment (start 251.968 101.346) (end 251.968 102.108) (width 1.5) (layer B.Cu) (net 11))
 (segment (start 218.186 99.822) (end 219.71 99.822) (width 1.5) (layer B.Cu) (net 11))
 (segment (start 226.568 98.552) (end 227.33 98.552) (width 1.5) (layer B.Cu) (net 11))
 (segment (start 227.33 98.552) (end 227.838 98.552) (width 1.5) (layer B.Cu) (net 11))
 (segment (start 225.044 100.076) (end 226.568 98.552) (width 1.5) (layer B.Cu) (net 11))
 (via (at 225.044 100.076) (size 1) (drill 0.6) (layers F.Cu B.Cu) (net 11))
 (segment (start 219.964 100.076) (end 225.044 100.076) (width 1.5) (layer F.Cu) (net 11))
 (segment (start 219.71 99.822) (end 219.964 100.076) (width 1.5) (layer F.Cu) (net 11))
 (via (at 219.71 99.822) (size 1) (drill 0.6) (layers F.Cu B.Cu) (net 11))
 (segment (start 221.234 115.316) (end 222.504 115.316) (width 1) (layer B.Cu) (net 11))
 (segment (start 221.234 115.316) (end 221.234 113.792) (width 1.5) (layer B.Cu) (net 11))
 (segment (start 218.186 110.744) (end 218.186 99.822) (width 1.5) (layer B.Cu) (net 11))
 (segment (start 221.234 113.792) (end 218.186 110.744) (width 1.5) (layer B.Cu) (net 11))
 (segment (start 218.186 99.822) (end 218.186 99.61) (width 1.5) (layer B.Cu) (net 11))
 (segment (start 218.186 99.61) (end 220.03 97.766) (width 1.5) (layer B.Cu) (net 11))
 (segment (start 242.062 105.41) (end 234.696 105.41) (width 1.5) (layer B.Cu) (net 13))
 (segment (start 251.968 115.316) (end 242.062 105.41) (width 1.5) (layer B.Cu) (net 13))
 (segment (start 251.968 124.968) (end 251.968 115.316) (width 1.5) (layer B.Cu) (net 13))
 (segment (start 232.664 103.378) (end 232.664 101.822) (width 1.5) (layer B.Cu) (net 13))
 (segment (start 234.696 105.41) (end 232.664 103.378) (width 1.5) (layer B.Cu) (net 13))
 (segment (start 240.792 107.95) (end 232.41 107.95) (width 1.5) (layer B.Cu) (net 14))
 (segment (start 249.428 116.586) (end 240.792 107.95) (width 1.5) (layer B.Cu) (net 14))
 (segment (start 249.428 124.968) (end 249.428 116.586) (width 1.5) (layer B.Cu) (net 14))
 (segment (start 228.092 103.632) (end 226.79 103.632) (width 1.5) (layer B.Cu) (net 14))
 (segment (start 232.41 107.95) (end 228.092 103.632) (width 1.5) (layer B.Cu) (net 14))
 (segment (start 230.312 97.766) (end 232.608 97.766) (width 1.5) (layer B.Cu) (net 10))
 (segment (start 232.608 97.766) (end 232.664 97.822) (width 1.5) (layer B.Cu) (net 10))
 (segment (start 222.504 102.394) (end 222.504 98.552) (width 1.5) (layer B.Cu) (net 12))
 (segment (start 222.504 98.552) (end 222.25 98.298) (width 1.5) (layer B.Cu) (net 12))
 (segment (start 222.25 98.298) (end 221.93 97.766) (width 1) (layer B.Cu) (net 12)))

